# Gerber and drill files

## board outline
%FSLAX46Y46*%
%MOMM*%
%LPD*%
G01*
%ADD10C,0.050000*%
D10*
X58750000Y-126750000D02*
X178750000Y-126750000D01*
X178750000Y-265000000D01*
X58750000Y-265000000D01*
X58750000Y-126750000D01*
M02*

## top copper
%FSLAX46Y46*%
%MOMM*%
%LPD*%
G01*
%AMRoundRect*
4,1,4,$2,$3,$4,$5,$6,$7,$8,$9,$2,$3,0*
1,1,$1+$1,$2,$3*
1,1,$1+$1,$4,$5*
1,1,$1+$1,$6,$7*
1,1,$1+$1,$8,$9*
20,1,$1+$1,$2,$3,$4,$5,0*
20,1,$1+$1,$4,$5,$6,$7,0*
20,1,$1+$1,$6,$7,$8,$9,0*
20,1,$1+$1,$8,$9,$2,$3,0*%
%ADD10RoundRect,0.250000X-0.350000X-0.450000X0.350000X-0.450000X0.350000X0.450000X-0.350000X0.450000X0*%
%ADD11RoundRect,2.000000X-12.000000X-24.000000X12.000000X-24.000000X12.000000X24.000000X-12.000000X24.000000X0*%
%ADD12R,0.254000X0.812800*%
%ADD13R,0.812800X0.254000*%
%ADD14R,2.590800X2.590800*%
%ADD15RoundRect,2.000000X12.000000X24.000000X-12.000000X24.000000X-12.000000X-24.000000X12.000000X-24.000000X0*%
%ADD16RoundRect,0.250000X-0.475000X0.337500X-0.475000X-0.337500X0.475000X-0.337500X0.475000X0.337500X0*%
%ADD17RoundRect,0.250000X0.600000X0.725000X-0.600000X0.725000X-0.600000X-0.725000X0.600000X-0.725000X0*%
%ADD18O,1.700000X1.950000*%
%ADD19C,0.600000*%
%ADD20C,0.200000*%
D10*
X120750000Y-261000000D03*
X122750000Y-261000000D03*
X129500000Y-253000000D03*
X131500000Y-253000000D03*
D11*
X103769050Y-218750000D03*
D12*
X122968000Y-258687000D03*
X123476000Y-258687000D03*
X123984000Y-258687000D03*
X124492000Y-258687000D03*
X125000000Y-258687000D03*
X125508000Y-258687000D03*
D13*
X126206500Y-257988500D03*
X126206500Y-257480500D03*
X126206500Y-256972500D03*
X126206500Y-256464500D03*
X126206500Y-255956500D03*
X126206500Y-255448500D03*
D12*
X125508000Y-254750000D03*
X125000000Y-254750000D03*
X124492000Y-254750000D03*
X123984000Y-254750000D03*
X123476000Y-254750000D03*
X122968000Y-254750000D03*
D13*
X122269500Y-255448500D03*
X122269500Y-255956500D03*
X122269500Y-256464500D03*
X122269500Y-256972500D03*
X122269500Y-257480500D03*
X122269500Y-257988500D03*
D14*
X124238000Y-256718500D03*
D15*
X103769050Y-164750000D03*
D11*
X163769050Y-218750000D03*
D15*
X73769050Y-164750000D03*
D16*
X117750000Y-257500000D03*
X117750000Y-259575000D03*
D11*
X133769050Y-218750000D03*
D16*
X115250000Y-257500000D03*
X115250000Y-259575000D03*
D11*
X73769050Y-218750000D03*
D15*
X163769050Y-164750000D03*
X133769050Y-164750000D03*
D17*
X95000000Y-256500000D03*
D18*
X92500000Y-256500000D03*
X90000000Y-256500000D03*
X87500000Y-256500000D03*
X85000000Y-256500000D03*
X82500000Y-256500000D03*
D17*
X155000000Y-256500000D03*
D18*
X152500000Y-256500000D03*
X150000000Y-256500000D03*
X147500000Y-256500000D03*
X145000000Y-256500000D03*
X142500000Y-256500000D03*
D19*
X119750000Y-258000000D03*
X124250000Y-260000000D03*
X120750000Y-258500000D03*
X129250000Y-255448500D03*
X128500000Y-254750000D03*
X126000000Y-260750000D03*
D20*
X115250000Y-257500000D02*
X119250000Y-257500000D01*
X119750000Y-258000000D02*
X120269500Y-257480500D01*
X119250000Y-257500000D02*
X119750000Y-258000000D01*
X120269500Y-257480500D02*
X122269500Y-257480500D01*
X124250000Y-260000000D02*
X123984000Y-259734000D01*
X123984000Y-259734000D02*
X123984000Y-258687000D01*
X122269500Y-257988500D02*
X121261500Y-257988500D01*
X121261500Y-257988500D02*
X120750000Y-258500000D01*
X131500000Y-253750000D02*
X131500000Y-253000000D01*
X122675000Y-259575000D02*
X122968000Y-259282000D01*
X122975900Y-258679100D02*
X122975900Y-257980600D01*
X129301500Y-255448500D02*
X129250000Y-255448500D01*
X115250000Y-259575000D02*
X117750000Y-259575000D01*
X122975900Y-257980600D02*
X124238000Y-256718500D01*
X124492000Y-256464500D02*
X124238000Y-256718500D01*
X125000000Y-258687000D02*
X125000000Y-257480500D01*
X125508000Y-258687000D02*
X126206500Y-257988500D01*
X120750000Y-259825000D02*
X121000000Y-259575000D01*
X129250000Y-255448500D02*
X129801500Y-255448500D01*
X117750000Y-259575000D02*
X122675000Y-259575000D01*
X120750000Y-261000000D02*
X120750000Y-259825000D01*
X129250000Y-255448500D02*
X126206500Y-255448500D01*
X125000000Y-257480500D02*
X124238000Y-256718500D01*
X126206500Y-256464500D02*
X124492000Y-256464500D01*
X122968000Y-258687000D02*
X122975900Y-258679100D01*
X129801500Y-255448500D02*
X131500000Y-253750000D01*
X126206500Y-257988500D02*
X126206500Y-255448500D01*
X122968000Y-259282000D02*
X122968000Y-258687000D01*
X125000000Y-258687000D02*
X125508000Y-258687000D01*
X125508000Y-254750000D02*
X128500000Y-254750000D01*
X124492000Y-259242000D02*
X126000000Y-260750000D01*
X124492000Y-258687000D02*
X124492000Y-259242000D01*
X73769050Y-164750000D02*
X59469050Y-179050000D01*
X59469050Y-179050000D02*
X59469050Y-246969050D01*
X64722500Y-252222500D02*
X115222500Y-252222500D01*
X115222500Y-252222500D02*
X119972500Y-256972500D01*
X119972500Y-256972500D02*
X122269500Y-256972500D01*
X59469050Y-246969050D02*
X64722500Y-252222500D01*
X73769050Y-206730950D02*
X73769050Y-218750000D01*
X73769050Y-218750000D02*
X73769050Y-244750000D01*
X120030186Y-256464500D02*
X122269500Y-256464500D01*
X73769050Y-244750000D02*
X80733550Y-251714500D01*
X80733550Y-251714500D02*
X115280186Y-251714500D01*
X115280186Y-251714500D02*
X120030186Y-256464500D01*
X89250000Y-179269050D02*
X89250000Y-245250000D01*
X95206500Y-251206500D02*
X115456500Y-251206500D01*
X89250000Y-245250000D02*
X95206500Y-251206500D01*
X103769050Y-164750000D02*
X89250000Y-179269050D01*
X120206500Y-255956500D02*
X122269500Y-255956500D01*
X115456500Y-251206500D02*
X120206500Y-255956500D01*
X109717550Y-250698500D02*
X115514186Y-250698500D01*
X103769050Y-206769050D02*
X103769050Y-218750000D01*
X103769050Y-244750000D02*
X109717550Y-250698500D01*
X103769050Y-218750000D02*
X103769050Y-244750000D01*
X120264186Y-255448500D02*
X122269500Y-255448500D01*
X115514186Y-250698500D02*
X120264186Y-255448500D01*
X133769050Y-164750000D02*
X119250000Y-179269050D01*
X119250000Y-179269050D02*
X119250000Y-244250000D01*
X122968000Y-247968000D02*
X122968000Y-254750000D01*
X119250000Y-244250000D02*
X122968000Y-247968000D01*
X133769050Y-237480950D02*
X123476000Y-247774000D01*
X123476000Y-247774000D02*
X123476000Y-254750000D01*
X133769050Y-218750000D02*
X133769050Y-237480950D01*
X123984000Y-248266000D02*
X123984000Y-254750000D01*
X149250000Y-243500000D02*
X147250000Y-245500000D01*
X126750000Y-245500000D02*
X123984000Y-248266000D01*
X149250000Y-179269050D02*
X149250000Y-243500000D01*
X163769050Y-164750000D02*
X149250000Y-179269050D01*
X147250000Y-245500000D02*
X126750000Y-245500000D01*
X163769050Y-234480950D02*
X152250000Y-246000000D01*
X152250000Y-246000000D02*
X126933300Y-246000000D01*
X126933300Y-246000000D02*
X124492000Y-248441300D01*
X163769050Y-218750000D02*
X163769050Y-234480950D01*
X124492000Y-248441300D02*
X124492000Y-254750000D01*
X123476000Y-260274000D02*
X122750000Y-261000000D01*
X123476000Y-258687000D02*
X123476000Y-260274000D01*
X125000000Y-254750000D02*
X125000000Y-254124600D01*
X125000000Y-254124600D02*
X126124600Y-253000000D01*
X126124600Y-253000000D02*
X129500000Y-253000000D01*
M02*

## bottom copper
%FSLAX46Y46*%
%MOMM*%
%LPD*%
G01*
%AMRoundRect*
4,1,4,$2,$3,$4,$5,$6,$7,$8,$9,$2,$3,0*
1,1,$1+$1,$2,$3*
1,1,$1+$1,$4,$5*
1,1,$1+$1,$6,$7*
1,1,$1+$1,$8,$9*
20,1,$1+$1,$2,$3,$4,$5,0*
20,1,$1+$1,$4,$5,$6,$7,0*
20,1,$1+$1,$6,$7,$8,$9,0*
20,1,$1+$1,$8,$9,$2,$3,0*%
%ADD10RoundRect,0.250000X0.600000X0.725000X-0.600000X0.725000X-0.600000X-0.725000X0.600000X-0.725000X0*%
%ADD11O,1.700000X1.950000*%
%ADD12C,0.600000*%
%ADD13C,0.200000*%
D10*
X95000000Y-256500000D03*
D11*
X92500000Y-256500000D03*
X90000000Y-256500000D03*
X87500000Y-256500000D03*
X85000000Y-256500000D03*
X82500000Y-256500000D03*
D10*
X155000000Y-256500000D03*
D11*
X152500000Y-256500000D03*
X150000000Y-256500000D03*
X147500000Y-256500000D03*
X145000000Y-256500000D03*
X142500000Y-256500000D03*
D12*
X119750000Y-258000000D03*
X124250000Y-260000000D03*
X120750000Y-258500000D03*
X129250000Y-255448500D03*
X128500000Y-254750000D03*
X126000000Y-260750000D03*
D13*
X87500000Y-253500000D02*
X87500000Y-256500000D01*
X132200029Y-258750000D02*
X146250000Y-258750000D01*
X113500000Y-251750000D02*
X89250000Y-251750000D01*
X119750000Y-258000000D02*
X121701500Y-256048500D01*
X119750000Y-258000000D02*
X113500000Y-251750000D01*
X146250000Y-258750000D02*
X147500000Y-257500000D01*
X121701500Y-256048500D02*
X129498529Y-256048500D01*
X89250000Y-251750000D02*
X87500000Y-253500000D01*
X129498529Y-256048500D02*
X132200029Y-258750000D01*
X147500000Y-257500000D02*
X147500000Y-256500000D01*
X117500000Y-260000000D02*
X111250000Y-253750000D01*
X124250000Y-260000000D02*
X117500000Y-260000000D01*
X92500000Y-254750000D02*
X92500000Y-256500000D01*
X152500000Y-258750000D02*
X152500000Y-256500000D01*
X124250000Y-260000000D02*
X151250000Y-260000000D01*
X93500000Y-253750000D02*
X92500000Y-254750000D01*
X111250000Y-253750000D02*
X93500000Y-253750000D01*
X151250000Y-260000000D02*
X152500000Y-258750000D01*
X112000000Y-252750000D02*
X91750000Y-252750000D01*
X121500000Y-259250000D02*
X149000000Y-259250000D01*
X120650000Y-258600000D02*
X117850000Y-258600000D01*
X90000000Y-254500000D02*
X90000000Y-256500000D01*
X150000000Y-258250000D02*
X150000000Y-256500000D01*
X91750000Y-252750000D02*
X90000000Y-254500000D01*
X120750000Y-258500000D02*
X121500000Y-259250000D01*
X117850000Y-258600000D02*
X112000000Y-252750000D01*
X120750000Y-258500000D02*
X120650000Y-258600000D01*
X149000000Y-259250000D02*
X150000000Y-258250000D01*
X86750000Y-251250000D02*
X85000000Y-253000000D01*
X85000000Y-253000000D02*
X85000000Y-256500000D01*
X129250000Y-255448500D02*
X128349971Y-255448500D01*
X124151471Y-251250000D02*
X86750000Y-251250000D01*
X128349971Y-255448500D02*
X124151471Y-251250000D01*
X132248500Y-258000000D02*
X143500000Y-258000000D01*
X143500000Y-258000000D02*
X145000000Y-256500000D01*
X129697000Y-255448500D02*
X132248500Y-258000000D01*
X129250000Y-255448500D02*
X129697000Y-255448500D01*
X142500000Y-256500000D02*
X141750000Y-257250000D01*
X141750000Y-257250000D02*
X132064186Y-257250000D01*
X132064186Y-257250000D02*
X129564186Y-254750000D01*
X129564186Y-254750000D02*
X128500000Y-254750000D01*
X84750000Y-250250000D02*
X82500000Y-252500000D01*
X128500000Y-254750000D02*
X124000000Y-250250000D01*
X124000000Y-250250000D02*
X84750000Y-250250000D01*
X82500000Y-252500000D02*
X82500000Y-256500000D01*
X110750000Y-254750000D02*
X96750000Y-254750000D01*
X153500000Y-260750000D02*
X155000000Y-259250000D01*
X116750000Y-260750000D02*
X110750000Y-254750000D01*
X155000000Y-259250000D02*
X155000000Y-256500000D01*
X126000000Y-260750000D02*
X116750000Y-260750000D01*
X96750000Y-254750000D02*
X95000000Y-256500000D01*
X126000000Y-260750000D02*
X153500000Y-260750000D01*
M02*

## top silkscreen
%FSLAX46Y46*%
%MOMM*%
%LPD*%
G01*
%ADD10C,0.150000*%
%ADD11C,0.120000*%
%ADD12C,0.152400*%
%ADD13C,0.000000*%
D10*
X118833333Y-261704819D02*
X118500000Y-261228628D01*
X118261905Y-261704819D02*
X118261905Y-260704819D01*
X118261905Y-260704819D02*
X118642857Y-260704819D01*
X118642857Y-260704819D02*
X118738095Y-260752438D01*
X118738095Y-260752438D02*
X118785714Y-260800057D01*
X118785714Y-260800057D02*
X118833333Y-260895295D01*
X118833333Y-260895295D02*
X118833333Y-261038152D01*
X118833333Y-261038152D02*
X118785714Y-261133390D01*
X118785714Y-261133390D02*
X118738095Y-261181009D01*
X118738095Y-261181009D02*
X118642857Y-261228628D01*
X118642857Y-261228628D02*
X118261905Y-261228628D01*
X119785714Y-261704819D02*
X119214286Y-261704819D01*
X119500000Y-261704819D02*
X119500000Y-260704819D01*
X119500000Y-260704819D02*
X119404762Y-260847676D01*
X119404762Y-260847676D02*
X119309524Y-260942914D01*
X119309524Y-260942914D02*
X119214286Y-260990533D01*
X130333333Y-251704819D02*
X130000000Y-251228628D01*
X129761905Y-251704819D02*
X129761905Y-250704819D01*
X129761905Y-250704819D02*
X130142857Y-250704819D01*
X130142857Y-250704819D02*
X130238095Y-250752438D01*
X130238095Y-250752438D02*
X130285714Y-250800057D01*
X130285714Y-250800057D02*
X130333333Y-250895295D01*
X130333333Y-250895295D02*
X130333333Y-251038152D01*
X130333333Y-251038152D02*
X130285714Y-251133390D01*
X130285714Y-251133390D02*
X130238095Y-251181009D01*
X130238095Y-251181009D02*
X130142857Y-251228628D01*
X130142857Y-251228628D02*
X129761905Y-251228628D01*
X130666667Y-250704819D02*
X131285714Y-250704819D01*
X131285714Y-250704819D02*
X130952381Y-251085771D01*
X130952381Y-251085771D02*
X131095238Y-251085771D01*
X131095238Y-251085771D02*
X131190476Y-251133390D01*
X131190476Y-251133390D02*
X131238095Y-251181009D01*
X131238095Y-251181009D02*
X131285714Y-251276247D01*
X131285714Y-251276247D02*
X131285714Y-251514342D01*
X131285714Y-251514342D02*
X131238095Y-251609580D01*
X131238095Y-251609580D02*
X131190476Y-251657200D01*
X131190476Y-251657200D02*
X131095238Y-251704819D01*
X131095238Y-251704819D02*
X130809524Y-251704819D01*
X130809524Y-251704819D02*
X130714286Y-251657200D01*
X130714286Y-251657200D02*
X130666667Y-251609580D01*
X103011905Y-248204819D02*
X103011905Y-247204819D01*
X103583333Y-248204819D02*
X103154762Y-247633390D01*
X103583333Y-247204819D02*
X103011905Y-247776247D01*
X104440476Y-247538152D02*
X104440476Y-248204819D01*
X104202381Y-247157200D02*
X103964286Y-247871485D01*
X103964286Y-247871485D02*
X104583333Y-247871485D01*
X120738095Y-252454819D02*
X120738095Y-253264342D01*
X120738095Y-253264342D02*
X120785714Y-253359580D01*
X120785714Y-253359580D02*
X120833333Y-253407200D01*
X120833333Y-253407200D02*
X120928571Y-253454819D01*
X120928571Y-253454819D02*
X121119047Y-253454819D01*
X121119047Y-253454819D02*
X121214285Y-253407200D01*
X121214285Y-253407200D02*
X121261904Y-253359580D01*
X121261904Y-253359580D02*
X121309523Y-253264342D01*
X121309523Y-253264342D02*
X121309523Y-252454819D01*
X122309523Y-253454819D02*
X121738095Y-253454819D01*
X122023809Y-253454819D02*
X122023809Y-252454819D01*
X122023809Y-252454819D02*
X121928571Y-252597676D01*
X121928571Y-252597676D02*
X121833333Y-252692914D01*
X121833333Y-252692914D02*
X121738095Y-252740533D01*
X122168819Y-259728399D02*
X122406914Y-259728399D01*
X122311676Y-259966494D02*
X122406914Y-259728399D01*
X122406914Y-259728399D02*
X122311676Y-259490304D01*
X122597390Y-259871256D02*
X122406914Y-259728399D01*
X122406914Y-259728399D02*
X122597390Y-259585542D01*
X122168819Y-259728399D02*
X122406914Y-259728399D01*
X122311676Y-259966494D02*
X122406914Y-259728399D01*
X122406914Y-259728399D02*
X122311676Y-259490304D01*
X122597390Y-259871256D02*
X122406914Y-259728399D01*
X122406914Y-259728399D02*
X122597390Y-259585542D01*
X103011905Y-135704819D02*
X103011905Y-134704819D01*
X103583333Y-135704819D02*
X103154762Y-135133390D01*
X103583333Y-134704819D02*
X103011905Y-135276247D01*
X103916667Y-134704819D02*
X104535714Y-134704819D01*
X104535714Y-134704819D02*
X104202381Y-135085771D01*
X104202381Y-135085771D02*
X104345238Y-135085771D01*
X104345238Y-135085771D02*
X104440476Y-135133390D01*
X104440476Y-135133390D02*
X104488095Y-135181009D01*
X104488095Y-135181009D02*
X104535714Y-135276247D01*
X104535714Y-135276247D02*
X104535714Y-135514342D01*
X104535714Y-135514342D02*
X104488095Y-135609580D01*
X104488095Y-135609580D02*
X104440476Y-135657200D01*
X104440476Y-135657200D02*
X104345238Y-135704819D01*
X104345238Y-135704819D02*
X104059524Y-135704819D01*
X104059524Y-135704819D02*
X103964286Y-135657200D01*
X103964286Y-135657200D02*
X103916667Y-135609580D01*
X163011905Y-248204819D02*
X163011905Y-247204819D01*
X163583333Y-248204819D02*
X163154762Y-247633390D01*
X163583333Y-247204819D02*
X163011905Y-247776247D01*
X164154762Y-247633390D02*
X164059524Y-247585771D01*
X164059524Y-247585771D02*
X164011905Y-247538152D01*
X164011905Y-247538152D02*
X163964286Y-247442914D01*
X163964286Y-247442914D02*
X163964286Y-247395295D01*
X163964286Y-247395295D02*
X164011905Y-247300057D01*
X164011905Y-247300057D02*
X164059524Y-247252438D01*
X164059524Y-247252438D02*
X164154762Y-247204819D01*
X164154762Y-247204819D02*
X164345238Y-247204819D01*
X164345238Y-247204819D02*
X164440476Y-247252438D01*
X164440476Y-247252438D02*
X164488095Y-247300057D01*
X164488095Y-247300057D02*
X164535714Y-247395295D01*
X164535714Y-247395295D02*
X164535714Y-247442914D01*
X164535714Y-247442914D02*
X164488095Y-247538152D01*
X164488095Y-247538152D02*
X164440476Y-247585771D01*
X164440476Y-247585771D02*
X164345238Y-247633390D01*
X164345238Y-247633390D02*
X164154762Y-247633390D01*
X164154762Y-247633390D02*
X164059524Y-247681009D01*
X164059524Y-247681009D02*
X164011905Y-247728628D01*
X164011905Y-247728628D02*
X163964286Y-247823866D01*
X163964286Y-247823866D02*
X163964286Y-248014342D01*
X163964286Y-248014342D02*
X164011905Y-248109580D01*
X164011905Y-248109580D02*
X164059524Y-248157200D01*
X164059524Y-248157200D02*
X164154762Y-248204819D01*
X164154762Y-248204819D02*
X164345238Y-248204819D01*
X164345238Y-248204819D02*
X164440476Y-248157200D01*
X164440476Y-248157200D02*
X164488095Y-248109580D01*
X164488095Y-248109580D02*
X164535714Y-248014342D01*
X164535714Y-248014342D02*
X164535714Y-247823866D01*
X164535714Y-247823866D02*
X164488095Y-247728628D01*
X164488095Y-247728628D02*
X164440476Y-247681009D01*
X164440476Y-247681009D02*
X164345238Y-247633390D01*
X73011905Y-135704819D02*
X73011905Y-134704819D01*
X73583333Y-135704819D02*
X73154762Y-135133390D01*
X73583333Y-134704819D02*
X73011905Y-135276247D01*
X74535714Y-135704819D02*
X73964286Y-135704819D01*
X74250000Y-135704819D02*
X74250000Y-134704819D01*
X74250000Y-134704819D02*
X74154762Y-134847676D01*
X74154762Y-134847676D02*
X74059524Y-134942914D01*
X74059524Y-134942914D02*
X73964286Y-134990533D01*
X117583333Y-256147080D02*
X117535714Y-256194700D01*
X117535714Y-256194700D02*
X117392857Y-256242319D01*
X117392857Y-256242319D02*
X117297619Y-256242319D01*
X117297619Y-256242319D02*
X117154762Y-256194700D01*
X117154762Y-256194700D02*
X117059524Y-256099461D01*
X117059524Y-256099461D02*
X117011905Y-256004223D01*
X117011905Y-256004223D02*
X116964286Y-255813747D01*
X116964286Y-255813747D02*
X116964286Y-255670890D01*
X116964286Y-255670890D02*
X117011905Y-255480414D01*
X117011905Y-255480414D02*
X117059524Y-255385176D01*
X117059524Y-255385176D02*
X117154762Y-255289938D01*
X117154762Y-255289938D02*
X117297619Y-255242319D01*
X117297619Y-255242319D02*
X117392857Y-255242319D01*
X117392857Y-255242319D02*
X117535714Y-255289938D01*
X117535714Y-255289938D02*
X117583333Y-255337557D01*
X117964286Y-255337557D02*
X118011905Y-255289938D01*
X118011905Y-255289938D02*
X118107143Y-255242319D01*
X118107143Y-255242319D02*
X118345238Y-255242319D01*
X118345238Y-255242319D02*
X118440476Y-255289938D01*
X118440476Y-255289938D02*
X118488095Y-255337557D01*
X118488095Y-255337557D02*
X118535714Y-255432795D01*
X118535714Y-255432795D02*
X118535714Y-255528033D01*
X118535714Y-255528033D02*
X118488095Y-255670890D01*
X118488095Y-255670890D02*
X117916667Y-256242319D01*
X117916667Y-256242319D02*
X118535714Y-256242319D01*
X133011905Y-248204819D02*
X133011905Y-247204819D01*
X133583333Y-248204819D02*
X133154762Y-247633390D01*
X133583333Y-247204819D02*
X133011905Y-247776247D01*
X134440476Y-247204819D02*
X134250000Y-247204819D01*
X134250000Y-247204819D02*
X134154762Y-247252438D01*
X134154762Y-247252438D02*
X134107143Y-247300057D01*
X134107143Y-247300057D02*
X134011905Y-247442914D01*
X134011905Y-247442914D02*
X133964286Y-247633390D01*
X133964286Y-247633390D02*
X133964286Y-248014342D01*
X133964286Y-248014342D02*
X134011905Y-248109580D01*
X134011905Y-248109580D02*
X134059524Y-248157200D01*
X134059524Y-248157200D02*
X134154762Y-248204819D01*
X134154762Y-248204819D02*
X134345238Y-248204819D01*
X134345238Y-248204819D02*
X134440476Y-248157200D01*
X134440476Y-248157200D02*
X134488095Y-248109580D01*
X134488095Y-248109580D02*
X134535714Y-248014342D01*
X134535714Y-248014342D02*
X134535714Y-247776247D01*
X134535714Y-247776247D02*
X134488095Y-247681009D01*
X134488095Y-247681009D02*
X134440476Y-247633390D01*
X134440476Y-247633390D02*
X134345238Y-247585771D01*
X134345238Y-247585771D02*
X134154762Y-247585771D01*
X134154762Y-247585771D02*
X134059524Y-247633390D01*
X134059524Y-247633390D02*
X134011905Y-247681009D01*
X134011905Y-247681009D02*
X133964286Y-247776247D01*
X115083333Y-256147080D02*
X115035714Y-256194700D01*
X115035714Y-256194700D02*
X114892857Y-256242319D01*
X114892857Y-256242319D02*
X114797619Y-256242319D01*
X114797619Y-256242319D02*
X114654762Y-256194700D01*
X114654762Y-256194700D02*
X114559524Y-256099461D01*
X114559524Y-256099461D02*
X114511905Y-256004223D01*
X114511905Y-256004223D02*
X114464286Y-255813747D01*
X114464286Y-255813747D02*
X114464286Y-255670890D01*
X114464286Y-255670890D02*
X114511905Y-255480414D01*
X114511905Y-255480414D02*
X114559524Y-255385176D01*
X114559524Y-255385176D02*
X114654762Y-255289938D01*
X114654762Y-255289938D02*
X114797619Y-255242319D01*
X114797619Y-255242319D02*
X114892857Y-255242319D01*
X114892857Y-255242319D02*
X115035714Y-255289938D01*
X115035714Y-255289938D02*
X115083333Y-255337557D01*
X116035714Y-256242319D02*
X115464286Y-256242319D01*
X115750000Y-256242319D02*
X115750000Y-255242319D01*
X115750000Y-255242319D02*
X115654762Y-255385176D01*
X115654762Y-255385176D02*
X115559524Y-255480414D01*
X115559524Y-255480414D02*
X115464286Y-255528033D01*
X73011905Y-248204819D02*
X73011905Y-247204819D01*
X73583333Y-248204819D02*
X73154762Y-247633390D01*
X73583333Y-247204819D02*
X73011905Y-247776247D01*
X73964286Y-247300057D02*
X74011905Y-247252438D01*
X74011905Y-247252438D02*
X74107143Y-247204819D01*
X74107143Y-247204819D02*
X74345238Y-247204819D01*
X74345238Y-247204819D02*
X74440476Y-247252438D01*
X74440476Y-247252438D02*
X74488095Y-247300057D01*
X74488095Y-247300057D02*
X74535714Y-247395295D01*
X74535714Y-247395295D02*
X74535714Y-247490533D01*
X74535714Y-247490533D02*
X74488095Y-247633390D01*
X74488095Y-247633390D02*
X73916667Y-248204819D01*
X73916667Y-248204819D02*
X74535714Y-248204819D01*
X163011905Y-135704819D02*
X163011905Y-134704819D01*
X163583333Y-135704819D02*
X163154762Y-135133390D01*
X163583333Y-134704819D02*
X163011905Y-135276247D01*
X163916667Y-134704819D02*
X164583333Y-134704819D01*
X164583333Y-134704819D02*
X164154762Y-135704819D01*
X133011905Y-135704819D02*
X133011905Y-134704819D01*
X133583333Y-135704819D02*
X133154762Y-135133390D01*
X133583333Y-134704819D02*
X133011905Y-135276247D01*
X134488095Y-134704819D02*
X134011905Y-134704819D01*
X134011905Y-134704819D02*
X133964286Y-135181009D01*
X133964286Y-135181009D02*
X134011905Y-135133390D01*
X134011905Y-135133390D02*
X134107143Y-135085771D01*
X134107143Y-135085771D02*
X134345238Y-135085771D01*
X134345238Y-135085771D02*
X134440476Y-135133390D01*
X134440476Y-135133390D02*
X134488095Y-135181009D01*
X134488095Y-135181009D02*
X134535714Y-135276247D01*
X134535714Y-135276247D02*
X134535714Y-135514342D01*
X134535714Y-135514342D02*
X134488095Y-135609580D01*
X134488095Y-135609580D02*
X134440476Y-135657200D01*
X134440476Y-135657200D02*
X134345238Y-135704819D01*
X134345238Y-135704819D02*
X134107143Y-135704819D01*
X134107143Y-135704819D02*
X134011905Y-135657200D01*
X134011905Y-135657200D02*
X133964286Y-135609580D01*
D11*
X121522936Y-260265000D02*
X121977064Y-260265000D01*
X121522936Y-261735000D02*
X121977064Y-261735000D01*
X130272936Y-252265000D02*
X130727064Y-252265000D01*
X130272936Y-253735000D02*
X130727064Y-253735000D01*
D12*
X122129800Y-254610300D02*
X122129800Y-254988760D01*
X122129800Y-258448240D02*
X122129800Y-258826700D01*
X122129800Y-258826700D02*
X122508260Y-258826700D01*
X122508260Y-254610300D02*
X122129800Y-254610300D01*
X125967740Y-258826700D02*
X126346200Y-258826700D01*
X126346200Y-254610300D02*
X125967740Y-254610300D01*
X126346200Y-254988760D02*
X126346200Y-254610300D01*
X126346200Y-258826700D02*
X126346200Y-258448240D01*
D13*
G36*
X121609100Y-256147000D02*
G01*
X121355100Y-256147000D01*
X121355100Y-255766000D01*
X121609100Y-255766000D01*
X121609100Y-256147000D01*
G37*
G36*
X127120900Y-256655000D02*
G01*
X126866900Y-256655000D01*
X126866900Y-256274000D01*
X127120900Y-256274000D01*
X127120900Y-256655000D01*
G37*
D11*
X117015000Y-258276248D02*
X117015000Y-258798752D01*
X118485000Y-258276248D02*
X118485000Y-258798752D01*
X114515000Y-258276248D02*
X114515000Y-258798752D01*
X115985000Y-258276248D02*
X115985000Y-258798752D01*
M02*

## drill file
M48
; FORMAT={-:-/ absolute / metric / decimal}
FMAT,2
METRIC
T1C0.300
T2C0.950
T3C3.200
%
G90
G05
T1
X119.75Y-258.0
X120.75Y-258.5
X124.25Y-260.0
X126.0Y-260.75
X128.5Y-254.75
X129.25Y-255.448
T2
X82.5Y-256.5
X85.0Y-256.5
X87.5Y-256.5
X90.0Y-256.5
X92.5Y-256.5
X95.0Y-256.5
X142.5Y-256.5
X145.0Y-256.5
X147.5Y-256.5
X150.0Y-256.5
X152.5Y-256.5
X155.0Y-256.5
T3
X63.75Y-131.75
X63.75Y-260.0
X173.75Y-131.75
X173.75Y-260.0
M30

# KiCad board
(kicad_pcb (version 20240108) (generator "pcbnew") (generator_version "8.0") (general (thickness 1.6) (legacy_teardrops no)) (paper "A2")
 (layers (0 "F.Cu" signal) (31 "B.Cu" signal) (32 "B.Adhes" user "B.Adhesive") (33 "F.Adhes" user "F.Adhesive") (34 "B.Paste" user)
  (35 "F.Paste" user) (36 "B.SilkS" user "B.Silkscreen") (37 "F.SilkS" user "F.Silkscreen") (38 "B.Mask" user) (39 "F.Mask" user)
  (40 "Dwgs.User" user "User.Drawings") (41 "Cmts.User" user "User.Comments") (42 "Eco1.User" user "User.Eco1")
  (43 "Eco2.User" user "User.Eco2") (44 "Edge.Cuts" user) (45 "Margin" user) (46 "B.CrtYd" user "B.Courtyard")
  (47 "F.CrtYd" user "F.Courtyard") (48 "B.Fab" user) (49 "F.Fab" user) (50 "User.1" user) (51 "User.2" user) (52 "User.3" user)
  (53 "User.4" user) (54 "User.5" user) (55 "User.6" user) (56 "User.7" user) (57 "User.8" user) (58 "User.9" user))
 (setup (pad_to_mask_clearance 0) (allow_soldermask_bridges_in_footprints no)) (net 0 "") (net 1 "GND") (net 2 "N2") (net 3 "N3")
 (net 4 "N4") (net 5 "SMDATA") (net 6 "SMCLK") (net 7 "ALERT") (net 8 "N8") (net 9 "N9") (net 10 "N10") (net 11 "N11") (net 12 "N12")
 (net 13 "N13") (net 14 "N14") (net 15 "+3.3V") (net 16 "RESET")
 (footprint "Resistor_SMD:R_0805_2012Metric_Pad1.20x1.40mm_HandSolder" (layer "F.Cu") (at 121.75 261)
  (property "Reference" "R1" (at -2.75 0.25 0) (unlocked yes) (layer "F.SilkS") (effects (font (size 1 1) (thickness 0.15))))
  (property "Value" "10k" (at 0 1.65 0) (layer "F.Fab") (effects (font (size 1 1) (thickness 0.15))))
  (fp_line (start -0.227064 -0.735) (end 0.227064 -0.735) (stroke (width 0.12) (type solid)) (layer "F.SilkS"))
  (fp_line (start -0.227064 0.735) (end 0.227064 0.735) (stroke (width 0.12) (type solid)) (layer "F.SilkS"))
  (pad "1" smd roundrect (at -1 0) (size 1.2 1.4) (layers "F.Cu" "F.Paste" "F.Mask") (roundrect_rratio 0.208333) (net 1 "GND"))
  (pad "2" smd roundrect (at 1 0) (size 1.2 1.4) (layers "F.Cu" "F.Paste" "F.Mask") (roundrect_rratio 0.208333) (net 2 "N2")))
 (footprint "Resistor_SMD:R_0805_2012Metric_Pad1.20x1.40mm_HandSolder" (layer "F.Cu") (at 130.5 253)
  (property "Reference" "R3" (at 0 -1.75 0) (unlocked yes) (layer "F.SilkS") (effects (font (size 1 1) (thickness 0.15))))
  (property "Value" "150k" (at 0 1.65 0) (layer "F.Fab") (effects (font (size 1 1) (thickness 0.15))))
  (fp_line (start -0.227064 -0.735) (end 0.227064 -0.735) (stroke (width 0.12) (type solid)) (layer "F.SilkS"))
  (fp_line (start -0.227064 0.735) (end 0.227064 0.735) (stroke (width 0.12) (type solid)) (layer "F.SilkS"))
  (pad "1" smd roundrect (at -1 0) (size 1.2 1.4) (layers "F.Cu" "F.Paste" "F.Mask") (roundrect_rratio 0.208333) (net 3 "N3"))
  (pad "2" smd roundrect (at 1 0) (size 1.2 1.4) (layers "F.Cu" "F.Paste" "F.Mask") (roundrect_rratio 0.208333) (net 1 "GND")))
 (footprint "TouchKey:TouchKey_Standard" (layer "F.Cu") (at 103.76905 218.75)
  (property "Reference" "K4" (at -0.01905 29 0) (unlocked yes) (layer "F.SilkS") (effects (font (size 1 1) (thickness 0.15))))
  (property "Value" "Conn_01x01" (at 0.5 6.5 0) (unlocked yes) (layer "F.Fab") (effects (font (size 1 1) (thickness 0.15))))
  (pad "1" smd roundrect (at 0 0) (size 28 52) (layers "F.Cu") (roundrect_rratio 0.07142857143) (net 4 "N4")))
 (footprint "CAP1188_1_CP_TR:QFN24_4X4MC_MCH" (layer "F.Cu") (at 124.238 256.7185 90)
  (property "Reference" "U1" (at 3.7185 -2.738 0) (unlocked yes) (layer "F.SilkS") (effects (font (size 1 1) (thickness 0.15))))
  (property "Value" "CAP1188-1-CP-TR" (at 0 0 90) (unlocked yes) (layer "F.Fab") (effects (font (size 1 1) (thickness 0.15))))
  (fp_line (start 2.1082 -2.1082) (end 1.72974 -2.1082) (stroke (width 0.1524) (type solid)) (layer "F.SilkS"))
  (fp_line (start -1.72974 -2.1082) (end -2.1082 -2.1082) (stroke (width 0.1524) (type solid)) (layer "F.SilkS"))
  (fp_line (start -2.1082 -2.1082) (end -2.1082 -1.72974) (stroke (width 0.1524) (type solid)) (layer "F.SilkS"))
  (fp_line (start 2.1082 -1.72974) (end 2.1082 -2.1082) (stroke (width 0.1524) (type solid)) (layer "F.SilkS"))
  (fp_line (start -2.1082 1.72974) (end -2.1082 2.1082) (stroke (width 0.1524) (type solid)) (layer "F.SilkS"))
  (fp_line (start 2.1082 2.1082) (end 2.1082 1.72974) (stroke (width 0.1524) (type solid)) (layer "F.SilkS"))
  (fp_line (start 1.72974 2.1082) (end 2.1082 2.1082) (stroke (width 0.1524) (type solid)) (layer "F.SilkS"))
  (fp_line (start -2.1082 2.1082) (end -1.72974 2.1082) (stroke (width 0.1524) (type solid)) (layer "F.SilkS"))
  (fp_poly
   (pts (xy 0.5715 -2.6289) (xy 0.5715 -2.8829) (xy 0.9525 -2.8829) (xy 0.9525 -2.6289)) (stroke (width 0) (type solid)) (fill solid)
   (layer "F.SilkS"))
  (fp_poly
   (pts (xy 0.0635 2.6289) (xy 0.0635 2.8829) (xy 0.4445 2.8829) (xy 0.4445 2.6289)) (stroke (width 0) (type solid)) (fill solid)
   (layer "F.SilkS"))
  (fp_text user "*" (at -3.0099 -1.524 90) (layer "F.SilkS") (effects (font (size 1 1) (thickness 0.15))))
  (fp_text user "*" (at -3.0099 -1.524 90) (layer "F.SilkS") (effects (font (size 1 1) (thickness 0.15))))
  (pad "1" smd rect (at -1.9685 -1.27 180) (size 0.254 0.8128) (layers "F.Cu" "F.Paste" "F.Mask") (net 1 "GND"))
  (pad "2" smd rect (at -1.9685 -0.762 180) (size 0.254 0.8128) (layers "F.Cu" "F.Paste" "F.Mask") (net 2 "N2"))
  (pad "3" smd rect (at -1.9685 -0.254 180) (size 0.254 0.8128) (layers "F.Cu" "F.Paste" "F.Mask") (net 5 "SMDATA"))
  (pad "4" smd rect (at -1.9685 0.254 180) (size 0.254 0.8128) (layers "F.Cu" "F.Paste" "F.Mask") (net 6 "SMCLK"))
  (pad "5" smd rect (at -1.9685 0.762 180) (size 0.254 0.8128) (layers "F.Cu" "F.Paste" "F.Mask") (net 1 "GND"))
  (pad "6" smd rect (at -1.9685 1.27 180) (size 0.254 0.8128) (layers "F.Cu" "F.Paste" "F.Mask") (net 1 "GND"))
  (pad "7" smd rect (at -1.27 1.9685 90) (size 0.254 0.8128) (layers "F.Cu" "F.Paste" "F.Mask") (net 1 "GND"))
  (pad "8" smd rect (at -0.762 1.9685 90) (size 0.254 0.8128) (layers "F.Cu" "F.Paste" "F.Mask") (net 1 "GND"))
  (pad "9" smd rect (at -0.254 1.9685 90) (size 0.254 0.8128) (layers "F.Cu" "F.Paste" "F.Mask") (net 1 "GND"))
  (pad "10" smd rect (at 0.254 1.9685 90) (size 0.254 0.8128) (layers "F.Cu" "F.Paste" "F.Mask") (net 1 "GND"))
  (pad "11" smd rect (at 0.762 1.9685 90) (size 0.254 0.8128) (layers "F.Cu" "F.Paste" "F.Mask") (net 1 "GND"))
  (pad "12" smd rect (at 1.27 1.9685 90) (size 0.254 0.8128) (layers "F.Cu" "F.Paste" "F.Mask") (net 1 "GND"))
  (pad "13" smd rect (at 1.9685 1.27 180) (size 0.254 0.8128) (layers "F.Cu" "F.Paste" "F.Mask") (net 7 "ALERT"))
  (pad "14" smd rect (at 1.9685 0.762 180) (size 0.254 0.8128) (layers "F.Cu" "F.Paste" "F.Mask") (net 3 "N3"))
  (pad "15" smd rect (at 1.9685 0.254 180) (size 0.254 0.8128) (layers "F.Cu" "F.Paste" "F.Mask") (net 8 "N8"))
  (pad "16" smd rect (at 1.9685 -0.254 180) (size 0.254 0.8128) (layers "F.Cu" "F.Paste" "F.Mask") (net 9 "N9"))
  (pad "17" smd rect (at 1.9685 -0.762 180) (size 0.254 0.8128) (layers "F.Cu" "F.Paste" "F.Mask") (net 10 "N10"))
  (pad "18" smd rect (at 1.9685 -1.27 180) (size 0.254 0.8128) (layers "F.Cu" "F.Paste" "F.Mask") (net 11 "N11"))
  (pad "19" smd rect (at 1.27 -1.9685 90) (size 0.254 0.8128) (layers "F.Cu" "F.Paste" "F.Mask") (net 4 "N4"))
  (pad "20" smd rect (at 0.762 -1.9685 90) (size 0.254 0.8128) (layers "F.Cu" "F.Paste" "F.Mask") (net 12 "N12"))
  (pad "21" smd rect (at 0.254 -1.9685 90) (size 0.254 0.8128) (layers "F.Cu" "F.Paste" "F.Mask") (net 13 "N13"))
  (pad "22" smd rect (at -0.254 -1.9685 90) (size 0.254 0.8128) (layers "F.Cu" "F.Paste" "F.Mask") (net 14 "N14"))
  (pad "23" smd rect (at -0.762 -1.9685 90) (size 0.254 0.8128) (layers "F.Cu" "F.Paste" "F.Mask") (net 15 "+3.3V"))
  (pad "24" smd rect (at -1.27 -1.9685 90) (size 0.254 0.8128) (layers "F.Cu" "F.Paste" "F.Mask") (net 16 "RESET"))
  (pad "25" smd rect (at 0 0 90) (size 2.5908 2.5908) (layers "F.Cu" "F.Paste" "F.Mask") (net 1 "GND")))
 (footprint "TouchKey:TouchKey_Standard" (layer "F.Cu") (at 103.76905 164.75 180)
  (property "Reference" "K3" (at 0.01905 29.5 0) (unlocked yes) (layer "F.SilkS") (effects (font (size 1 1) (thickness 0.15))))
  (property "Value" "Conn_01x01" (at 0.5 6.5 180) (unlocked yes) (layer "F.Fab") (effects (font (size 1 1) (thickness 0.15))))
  (pad "1" smd roundrect (at 0 0 180) (size 28 52) (layers "F.Cu") (roundrect_rratio 0.07142857143) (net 12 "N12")))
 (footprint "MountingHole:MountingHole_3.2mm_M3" (layer "F.Cu") (at 173.75 131.75)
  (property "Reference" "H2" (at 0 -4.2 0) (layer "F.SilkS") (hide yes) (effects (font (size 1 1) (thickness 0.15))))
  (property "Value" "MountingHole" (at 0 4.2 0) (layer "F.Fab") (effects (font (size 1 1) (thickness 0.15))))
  (pad "" np_thru_hole circle (at 0 0) (size 3.2 3.2) (drill 3.2) (layers "*.Cu" "*.Mask")))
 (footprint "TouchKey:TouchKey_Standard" (layer "F.Cu") (at 163.76905 218.75)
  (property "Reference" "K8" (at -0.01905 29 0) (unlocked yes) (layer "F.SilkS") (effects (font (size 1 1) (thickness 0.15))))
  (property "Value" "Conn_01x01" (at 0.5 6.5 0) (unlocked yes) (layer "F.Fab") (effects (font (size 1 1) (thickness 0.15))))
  (pad "1" smd roundrect (at 0 0) (size 28 52) (layers "F.Cu") (roundrect_rratio 0.07142857143) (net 8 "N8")))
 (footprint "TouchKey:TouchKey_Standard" (layer "F.Cu") (at 73.76905 164.75 180)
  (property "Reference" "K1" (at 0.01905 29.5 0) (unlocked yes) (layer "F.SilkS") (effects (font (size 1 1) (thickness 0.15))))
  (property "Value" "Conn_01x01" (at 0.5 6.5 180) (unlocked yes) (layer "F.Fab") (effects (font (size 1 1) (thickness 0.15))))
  (pad "1" smd roundrect (at 0 0 180) (size 28 52) (layers "F.Cu") (roundrect_rratio 0.07142857143) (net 14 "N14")))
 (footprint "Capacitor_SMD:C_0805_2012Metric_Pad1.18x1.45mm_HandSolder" (layer "F.Cu") (at 117.75 258.5375 -90)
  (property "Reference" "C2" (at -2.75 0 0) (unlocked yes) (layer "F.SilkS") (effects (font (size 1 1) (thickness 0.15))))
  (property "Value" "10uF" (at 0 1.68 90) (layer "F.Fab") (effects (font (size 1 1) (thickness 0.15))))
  (fp_line (start -0.261252 0.735) (end 0.261252 0.735) (stroke (width 0.12) (type solid)) (layer "F.SilkS"))
  (fp_line (start -0.261252 -0.735) (end 0.261252 -0.735) (stroke (width 0.12) (type solid)) (layer "F.SilkS"))
  (pad "1" smd roundrect (at -1.0375 0 270) (size 1.175 1.45) (layers "F.Cu" "F.Paste" "F.Mask") (roundrect_rratio 0.212766)
   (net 15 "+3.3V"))
  (pad "2" smd roundrect (at 1.0375 0 270) (size 1.175 1.45) (layers "F.Cu" "F.Paste" "F.Mask") (roundrect_rratio 0.212766) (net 1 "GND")))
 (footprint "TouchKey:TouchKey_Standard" (layer "F.Cu") (at 133.76905 218.75)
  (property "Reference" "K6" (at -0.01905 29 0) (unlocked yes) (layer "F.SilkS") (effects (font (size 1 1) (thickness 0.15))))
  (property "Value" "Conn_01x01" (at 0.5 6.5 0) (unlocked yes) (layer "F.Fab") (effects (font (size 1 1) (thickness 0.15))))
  (pad "1" smd roundrect (at 0 0) (size 28 52) (layers "F.Cu") (roundrect_rratio 0.07142857143) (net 10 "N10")))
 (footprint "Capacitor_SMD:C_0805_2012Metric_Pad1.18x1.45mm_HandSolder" (layer "F.Cu") (at 115.25 258.5375 -90)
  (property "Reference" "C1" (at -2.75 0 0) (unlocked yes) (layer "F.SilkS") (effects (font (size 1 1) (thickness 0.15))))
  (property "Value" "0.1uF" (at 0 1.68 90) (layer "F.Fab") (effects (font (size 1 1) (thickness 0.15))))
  (fp_line (start -0.261252 0.735) (end 0.261252 0.735) (stroke (width 0.12) (type solid)) (layer "F.SilkS"))
  (fp_line (start -0.261252 -0.735) (end 0.261252 -0.735) (stroke (width 0.12) (type solid)) (layer "F.SilkS"))
  (pad "1" smd roundrect (at -1.0375 0 270) (size 1.175 1.45) (layers "F.Cu" "F.Paste" "F.Mask") (roundrect_rratio 0.212766)
   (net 15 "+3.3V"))
  (pad "2" smd roundrect (at 1.0375 0 270) (size 1.175 1.45) (layers "F.Cu" "F.Paste" "F.Mask") (roundrect_rratio 0.212766) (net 1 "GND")))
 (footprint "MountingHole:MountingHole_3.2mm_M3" (layer "F.Cu") (at 63.75 260)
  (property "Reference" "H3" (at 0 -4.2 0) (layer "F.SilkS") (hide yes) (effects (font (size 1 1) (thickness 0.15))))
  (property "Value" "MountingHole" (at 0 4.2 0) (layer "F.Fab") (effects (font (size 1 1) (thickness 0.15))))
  (pad "" np_thru_hole circle (at 0 0) (size 3.2 3.2) (drill 3.2) (layers "*.Cu" "*.Mask")))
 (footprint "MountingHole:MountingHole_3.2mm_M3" (layer "F.Cu") (at 63.75 131.75)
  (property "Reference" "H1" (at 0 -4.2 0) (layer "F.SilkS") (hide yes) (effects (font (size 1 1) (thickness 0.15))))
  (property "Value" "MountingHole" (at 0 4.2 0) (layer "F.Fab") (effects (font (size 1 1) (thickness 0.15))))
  (pad "" np_thru_hole circle (at 0 0) (size 3.2 3.2) (drill 3.2) (layers "*.Cu" "*.Mask")))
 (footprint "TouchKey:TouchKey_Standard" (layer "F.Cu") (at 73.76905 218.75)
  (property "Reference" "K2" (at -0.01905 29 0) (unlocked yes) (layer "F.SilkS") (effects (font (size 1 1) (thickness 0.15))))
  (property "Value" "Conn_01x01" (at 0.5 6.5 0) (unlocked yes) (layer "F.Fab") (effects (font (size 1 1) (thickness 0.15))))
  (pad "1" smd roundrect (at 0 0) (size 28 52) (layers "F.Cu") (roundrect_rratio 0.07142857143) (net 13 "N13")))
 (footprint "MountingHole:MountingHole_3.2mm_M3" (layer "F.Cu") (at 173.75 260)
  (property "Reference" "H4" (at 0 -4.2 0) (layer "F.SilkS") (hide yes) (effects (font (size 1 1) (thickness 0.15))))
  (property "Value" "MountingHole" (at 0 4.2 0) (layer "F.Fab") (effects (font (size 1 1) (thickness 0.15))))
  (pad "" np_thru_hole circle (at 0 0) (size 3.2 3.2) (drill 3.2) (layers "*.Cu" "*.Mask")))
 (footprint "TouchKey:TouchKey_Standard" (layer "F.Cu") (at 163.76905 164.75 180)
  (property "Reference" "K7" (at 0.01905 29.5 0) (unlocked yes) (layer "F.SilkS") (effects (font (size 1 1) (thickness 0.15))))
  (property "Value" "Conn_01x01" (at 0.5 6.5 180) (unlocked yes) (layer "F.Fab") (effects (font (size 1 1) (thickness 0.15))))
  (pad "1" smd roundrect (at 0 0 180) (size 28 52) (layers "F.Cu") (roundrect_rratio 0.07142857143) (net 9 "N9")))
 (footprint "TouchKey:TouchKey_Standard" (layer "F.Cu") (at 133.76905 164.75 180)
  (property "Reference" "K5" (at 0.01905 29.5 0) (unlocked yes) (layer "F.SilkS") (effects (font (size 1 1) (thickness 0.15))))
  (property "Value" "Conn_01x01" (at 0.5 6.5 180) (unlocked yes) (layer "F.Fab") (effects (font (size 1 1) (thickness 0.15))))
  (pad "1" smd roundrect (at 0 0 180) (size 28 52) (layers "F.Cu") (roundrect_rratio 0.07142857143) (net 11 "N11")))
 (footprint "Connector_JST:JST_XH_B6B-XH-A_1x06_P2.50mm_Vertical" (layer "B.Cu") (at 95 256.5 180)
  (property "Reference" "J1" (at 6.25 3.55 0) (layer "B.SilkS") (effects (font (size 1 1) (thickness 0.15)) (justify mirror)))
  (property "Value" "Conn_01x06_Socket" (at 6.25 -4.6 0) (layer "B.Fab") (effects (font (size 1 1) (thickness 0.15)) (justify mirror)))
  (pad "1" thru_hole roundrect (at 0 0 180) (size 1.7 1.95) (drill 0.95) (layers "*.Cu" "*.Mask") (remove_unused_layers no)
   (roundrect_rratio 0.147059) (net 6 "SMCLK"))
  (pad "2" thru_hole oval (at 2.5 0 180) (size 1.7 1.95) (drill 0.95) (layers "*.Cu" "*.Mask") (remove_unused_layers no) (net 5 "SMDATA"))
  (pad "3" thru_hole oval (at 5 0 180) (size 1.7 1.95) (drill 0.95) (layers "*.Cu" "*.Mask") (remove_unused_layers no) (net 16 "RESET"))
  (pad "4" thru_hole oval (at 7.5 0 180) (size 1.7 1.95) (drill 0.95) (layers "*.Cu" "*.Mask") (remove_unused_layers no) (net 15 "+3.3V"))
  (pad "5" thru_hole oval (at 10 0 180) (size 1.7 1.95) (drill 0.95) (layers "*.Cu" "*.Mask") (remove_unused_layers no) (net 1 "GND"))
  (pad "6" thru_hole oval (at 12.5 0 180) (size 1.7 1.95) (drill 0.95) (layers "*.Cu" "*.Mask") (remove_unused_layers no) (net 7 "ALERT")))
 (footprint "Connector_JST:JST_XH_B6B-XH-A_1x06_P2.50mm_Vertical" (layer "B.Cu") (at 155 256.5 180)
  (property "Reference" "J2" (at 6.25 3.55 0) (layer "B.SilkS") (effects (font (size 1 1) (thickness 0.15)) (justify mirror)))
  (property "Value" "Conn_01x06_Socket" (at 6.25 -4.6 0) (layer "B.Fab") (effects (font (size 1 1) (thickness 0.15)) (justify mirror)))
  (pad "1" thru_hole roundrect (at 0 0 180) (size 1.7 1.95) (drill 0.95) (layers "*.Cu" "*.Mask") (remove_unused_layers no)
   (roundrect_rratio 0.147059) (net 6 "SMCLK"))
  (pad "2" thru_hole oval (at 2.5 0 180) (size 1.7 1.95) (drill 0.95) (layers "*.Cu" "*.Mask") (remove_unused_layers no) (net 5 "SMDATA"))
  (pad "3" thru_hole oval (at 5 0 180) (size 1.7 1.95) (drill 0.95) (layers "*.Cu" "*.Mask") (remove_unused_layers no) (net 16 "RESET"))
  (pad "4" thru_hole oval (at 7.5 0 180) (size 1.7 1.95) (drill 0.95) (layers "*.Cu" "*.Mask") (remove_unused_layers no) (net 15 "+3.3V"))
  (pad "5" thru_hole oval (at 10 0 180) (size 1.7 1.95) (drill 0.95) (layers "*.Cu" "*.Mask") (remove_unused_layers no) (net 1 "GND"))
  (pad "6" thru_hole oval (at 12.5 0 180) (size 1.7 1.95) (drill 0.95) (layers "*.Cu" "*.Mask") (remove_unused_layers no) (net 7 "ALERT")))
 (gr_rect (start 58.75 126.75) (end 178.75 265) (stroke (width 0.05) (type default)) (fill none) (layer "Edge.Cuts"))
 (segment (start 115.25 257.5) (end 119.25 257.5) (width 0.2) (layer "F.Cu") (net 15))
 (segment (start 119.75 258) (end 120.2695 257.4805) (width 0.2) (layer "F.Cu") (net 15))
 (segment (start 119.25 257.5) (end 119.75 258) (width 0.2) (layer "F.Cu") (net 15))
 (segment (start 120.2695 257.4805) (end 122.2695 257.4805) (width 0.2) (layer "F.Cu") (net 15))
 (via (at 119.75 258) (size 0.6) (drill 0.3) (layers "F.Cu" "B.Cu") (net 15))
 (segment (start 87.5 253.5) (end 87.5 256.5) (width 0.2) (layer "B.Cu") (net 15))
 (segment (start 132.200029 258.75) (end 146.25 258.75) (width 0.2) (layer "B.Cu") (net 15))
 (segment (start 113.5 251.75) (end 89.25 251.75) (width 0.2) (layer "B.Cu") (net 15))
 (segment (start 119.75 258) (end 121.7015 256.0485) (width 0.2) (layer "B.Cu") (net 15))
 (segment (start 119.75 258) (end 113.5 251.75) (width 0.2) (layer "B.Cu") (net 15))
 (segment (start 146.25 258.75) (end 147.5 257.5) (width 0.2) (layer "B.Cu") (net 15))
 (segment (start 121.7015 256.0485) (end 129.498529 256.0485) (width 0.2) (layer "B.Cu") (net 15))
 (segment (start 89.25 251.75) (end 87.5 253.5) (width 0.2) (layer "B.Cu") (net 15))
 (segment (start 129.498529 256.0485) (end 132.200029 258.75) (width 0.2) (layer "B.Cu") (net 15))
 (segment (start 147.5 257.5) (end 147.5 256.5) (width 0.2) (layer "B.Cu") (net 15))
 (segment (start 124.25 260) (end 123.984 259.734) (width 0.2) (layer "F.Cu") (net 5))
 (segment (start 123.984 259.734) (end 123.984 258.687) (width 0.2) (layer "F.Cu") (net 5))
 (via (at 124.25 260) (size 0.6) (drill 0.3) (layers "F.Cu" "B.Cu") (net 5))
 (segment (start 117.5 260) (end 111.25 253.75) (width 0.2) (layer "B.Cu") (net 5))
 (segment (start 124.25 260) (end 117.5 260) (width 0.2) (layer "B.Cu") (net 5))
 (segment (start 92.5 254.75) (end 92.5 256.5) (width 0.2) (layer "B.Cu") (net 5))
 (segment (start 152.5 258.75) (end 152.5 256.5) (width 0.2) (layer "B.Cu") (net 5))
 (segment (start 124.25 260) (end 151.25 260) (width 0.2) (layer "B.Cu") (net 5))
 (segment (start 93.5 253.75) (end 92.5 254.75) (width 0.2) (layer "B.Cu") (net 5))
 (segment (start 111.25 253.75) (end 93.5 253.75) (width 0.2) (layer "B.Cu") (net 5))
 (segment (start 151.25 260) (end 152.5 258.75) (width 0.2) (layer "B.Cu") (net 5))
 (segment (start 122.2695 257.9885) (end 121.2615 257.9885) (width 0.2) (layer "F.Cu") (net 16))
 (segment (start 121.2615 257.9885) (end 120.75 258.5) (width 0.2) (layer "F.Cu") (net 16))
 (via (at 120.75 258.5) (size 0.6) (drill 0.3) (layers "F.Cu" "B.Cu") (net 16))
 (segment (start 112 252.75) (end 91.75 252.75) (width 0.2) (layer "B.Cu") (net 16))
 (segment (start 121.5 259.25) (end 149 259.25) (width 0.2) (layer "B.Cu") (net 16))
 (segment (start 120.65 258.6) (end 117.85 258.6) (width 0.2) (layer "B.Cu") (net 16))
 (segment (start 90 254.5) (end 90 256.5) (width 0.2) (layer "B.Cu") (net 16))
 (segment (start 150 258.25) (end 150 256.5) (width 0.2) (layer "B.Cu") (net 16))
 (segment (start 91.75 252.75) (end 90 254.5) (width 0.2) (layer "B.Cu") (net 16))
 (segment (start 120.75 258.5) (end 121.5 259.25) (width 0.2) (layer "B.Cu") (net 16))
 (segment (start 117.85 258.6) (end 112 252.75) (width 0.2) (layer "B.Cu") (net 16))
 (segment (start 120.75 258.5) (end 120.65 258.6) (width 0.2) (layer "B.Cu") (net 16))
 (segment (start 149 259.25) (end 150 258.25) (width 0.2) (layer "B.Cu") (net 16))
 (segment (start 131.5 253.75) (end 131.5 253) (width 0.2) (layer "F.Cu") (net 1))
 (segment (start 122.675 259.575) (end 122.968 259.282) (width 0.2) (layer "F.Cu") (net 1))
 (segment (start 122.9759 258.6791) (end 122.9759 257.9806) (width 0.2) (layer "F.Cu") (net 1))
 (segment (start 129.3015 255.4485) (end 129.25 255.4485) (width 0.2) (layer "F.Cu") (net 1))
 (segment (start 115.25 259.575) (end 117.75 259.575) (width 0.2) (layer "F.Cu") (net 1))
 (segment (start 122.9759 257.9806) (end 124.238 256.7185) (width 0.2) (layer "F.Cu") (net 1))
 (segment (start 124.492 256.4645) (end 124.238 256.7185) (width 0.2) (layer "F.Cu") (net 1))
 (segment (start 125 258.687) (end 125 257.4805) (width 0.2) (layer "F.Cu") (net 1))
 (segment (start 125.508 258.687) (end 126.2065 257.9885) (width 0.2) (layer "F.Cu") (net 1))
 (segment (start 120.75 259.825) (end 121 259.575) (width 0.2) (layer "F.Cu") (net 1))
 (segment (start 129.25 255.4485) (end 129.8015 255.4485) (width 0.2) (layer "F.Cu") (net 1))
 (segment (start 117.75 259.575) (end 122.675 259.575) (width 0.2) (layer "F.Cu") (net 1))
 (segment (start 120.75 261) (end 120.75 259.825) (width 0.2) (layer "F.Cu") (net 1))
 (segment (start 129.25 255.4485) (end 126.2065 255.4485) (width 0.2) (layer "F.Cu") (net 1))
 (segment (start 125 257.4805) (end 124.238 256.7185) (width 0.2) (layer "F.Cu") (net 1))
 (segment (start 126.2065 256.4645) (end 124.492 256.4645) (width 0.2) (layer "F.Cu") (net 1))
 (segment (start 122.968 258.687) (end 122.9759 258.6791) (width 0.2) (layer "F.Cu") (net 1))
 (segment (start 129.8015 255.4485) (end 131.5 253.75) (width 0.2) (layer "F.Cu") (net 1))
 (segment (start 126.2065 257.9885) (end 126.2065 255.4485) (width 0.2) (layer "F.Cu") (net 1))
 (segment (start 122.968 259.282) (end 122.968 258.687) (width 0.2) (layer "F.Cu") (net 1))
 (segment (start 125 258.687) (end 125.508 258.687) (width 0.2) (layer "F.Cu") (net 1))
 (via (at 129.25 255.4485) (size 0.6) (drill 0.3) (layers "F.Cu" "B.Cu") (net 1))
 (segment (start 86.75 251.25) (end 85 253) (width 0.2) (layer "B.Cu") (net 1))
 (segment (start 85 253) (end 85 256.5) (width 0.2) (layer "B.Cu") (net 1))
 (segment (start 129.25 255.4485) (end 128.349971 255.4485) (width 0.2) (layer "B.Cu") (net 1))
 (segment (start 124.151471 251.25) (end 86.75 251.25) (width 0.2) (layer "B.Cu") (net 1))
 (segment (start 128.349971 255.4485) (end 124.151471 251.25) (width 0.2) (layer "B.Cu") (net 1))
 (segment (start 132.2485 258) (end 143.5 258) (width 0.2) (layer "B.Cu") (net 1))
 (segment (start 143.5 258) (end 145 256.5) (width 0.2) (layer "B.Cu") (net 1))
 (segment (start 129.697 255.4485) (end 132.2485 258) (width 0.2) (layer "B.Cu") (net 1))
 (segment (start 129.25 255.4485) (end 129.697 255.4485) (width 0.2) (layer "B.Cu") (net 1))
 (segment (start 125.508 254.75) (end 128.5 254.75) (width 0.2) (layer "F.Cu") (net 7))
 (via (at 128.5 254.75) (size 0.6) (drill 0.3) (layers "F.Cu" "B.Cu") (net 7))
 (segment (start 142.5 256.5) (end 141.75 257.25) (width 0.2) (layer "B.Cu") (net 7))
 (segment (start 141.75 257.25) (end 132.064186 257.25) (width 0.2) (layer "B.Cu") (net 7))
 (segment (start 132.064186 257.25) (end 129.564186 254.75) (width 0.2) (layer "B.Cu") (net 7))
 (segment (start 129.564186 254.75) (end 128.5 254.75) (width 0.2) (layer "B.Cu") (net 7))
 (segment (start 84.75 250.25) (end 82.5 252.5) (width 0.2) (layer "B.Cu") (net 7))
 (segment (start 128.5 254.75) (end 124 250.25) (width 0.2) (layer "B.Cu") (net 7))
 (segment (start 124 250.25) (end 84.75 250.25) (width 0.2) (layer "B.Cu") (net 7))
 (segment (start 82.5 252.5) (end 82.5 256.5) (width 0.2) (layer "B.Cu") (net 7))
 (segment (start 124.492 259.242) (end 126 260.75) (width 0.2) (layer "F.Cu") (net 6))
 (segment (start 124.492 258.687) (end 124.492 259.242) (width 0.2) (layer "F.Cu") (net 6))
 (via (at 126 260.75) (size 0.6) (drill 0.3) (layers "F.Cu" "B.Cu") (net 6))
 (segment (start 110.75 254.75) (end 96.75 254.75) (width 0.2) (layer "B.Cu") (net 6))
 (segment (start 153.5 260.75) (end 155 259.25) (width 0.2) (layer "B.Cu") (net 6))
 (segment (start 116.75 260.75) (end 110.75 254.75) (width 0.2) (layer "B.Cu") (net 6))
 (segment (start 155 259.25) (end 155 256.5) (width 0.2) (layer "B.Cu") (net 6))
 (segment (start 126 260.75) (end 116.75 260.75) (width 0.2) (layer "B.Cu") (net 6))
 (segment (start 96.75 254.75) (end 95 256.5) (width 0.2) (layer "B.Cu") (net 6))
 (segment (start 126 260.75) (end 153.5 260.75) (width 0.2) (layer "B.Cu") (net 6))
 (segment (start 73.76905 164.75) (end 59.46905 179.05) (width 0.2) (layer "F.Cu") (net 14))
 (segment (start 59.46905 179.05) (end 59.46905 246.96905) (width 0.2) (layer "F.Cu") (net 14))
 (segment (start 64.7225 252.2225) (end 115.2225 252.2225) (width 0.2) (layer "F.Cu") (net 14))
 (segment (start 115.2225 252.2225) (end 119.9725 256.9725) (width 0.2) (layer "F.Cu") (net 14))
 (segment (start 119.9725 256.9725) (end 122.2695 256.9725) (width 0.2) (layer "F.Cu") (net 14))
 (segment (start 59.46905 246.96905) (end 64.7225 252.2225) (width 0.2) (layer "F.Cu") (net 14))
 (segment (start 73.76905 206.73095) (end 73.76905 218.75) (width 0.2) (layer "F.Cu") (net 13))
 (segment (start 73.76905 218.75) (end 73.76905 244.75) (width 0.2) (layer "F.Cu") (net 13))
 (segment (start 120.030186 256.4645) (end 122.2695 256.4645) (width 0.2) (layer "F.Cu") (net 13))
 (segment (start 73.76905 244.75) (end 80.73355 251.7145) (width 0.2) (layer "F.Cu") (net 13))
 (segment (start 80.73355 251.7145) (end 115.280186 251.7145) (width 0.2) (layer "F.Cu") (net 13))
 (segment (start 115.280186 251.7145) (end 120.030186 256.4645) (width 0.2) (layer "F.Cu") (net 13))
 (segment (start 89.25 179.26905) (end 89.25 245.25) (width 0.2) (layer "F.Cu") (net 12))
 (segment (start 95.2065 251.2065) (end 115.4565 251.2065) (width 0.2) (layer "F.Cu") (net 12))
 (segment (start 89.25 245.25) (end 95.2065 251.2065) (width 0.2) (layer "F.Cu") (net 12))
 (segment (start 103.76905 164.75) (end 89.25 179.26905) (width 0.2) (layer "F.Cu") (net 12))
 (segment (start 120.2065 255.9565) (end 122.2695 255.9565) (width 0.2) (layer "F.Cu") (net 12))
 (segment (start 115.4565 251.2065) (end 120.2065 255.9565) (width 0.2) (layer "F.Cu") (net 12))
 (segment (start 109.71755 250.6985) (end 115.514186 250.6985) (width 0.2) (layer "F.Cu") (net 4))
 (segment (start 103.76905 206.76905) (end 103.76905 218.75) (width 0.2) (layer "F.Cu") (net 4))
 (segment (start 103.76905 244.75) (end 109.71755 250.6985) (width 0.2) (layer "F.Cu") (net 4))
 (segment (start 103.76905 218.75) (end 103.76905 244.75) (width 0.2) (layer "F.Cu") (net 4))
 (segment (start 120.264186 255.4485) (end 122.2695 255.4485) (width 0.2) (layer "F.Cu") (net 4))
 (segment (start 115.514186 250.6985) (end 120.264186 255.4485) (width 0.2) (layer "F.Cu") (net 4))
 (segment (start 133.76905 164.75) (end 119.25 179.26905) (width 0.2) (layer "F.Cu") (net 11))
 (segment (start 119.25 179.26905) (end 119.25 244.25) (width 0.2) (layer "F.Cu") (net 11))
 (segment (start 122.968 247.968) (end 122.968 254.75) (width 0.2) (layer "F.Cu") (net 11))
 (segment (start 119.25 244.25) (end 122.968 247.968) (width 0.2) (layer "F.Cu") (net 11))
 (segment (start 133.76905 237.48095) (end 123.476 247.774) (width 0.2) (layer "F.Cu") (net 10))
 (segment (start 123.476 247.774) (end 123.476 254.75) (width 0.2) (layer "F.Cu") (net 10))
 (segment (start 133.76905 218.75) (end 133.76905 237.48095) (width 0.2) (layer "F.Cu") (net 10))
 (segment (start 123.984 248.266) (end 123.984 254.75) (width 0.2) (layer "F.Cu") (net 9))
 (segment (start 149.25 243.5) (end 147.25 245.5) (width 0.2) (layer "F.Cu") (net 9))
 (segment (start 126.75 245.5) (end 123.984 248.266) (width 0.2) (layer "F.Cu") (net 9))
 (segment (start 149.25 179.26905) (end 149.25 243.5) (width 0.2) (layer "F.Cu") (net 9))
 (segment (start 163.76905 164.75) (end 149.25 179.26905) (width 0.2) (layer "F.Cu") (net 9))
 (segment (start 147.25 245.5) (end 126.75 245.5) (width 0.2) (layer "F.Cu") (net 9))
 (segment (start 163.76905 234.48095) (end 152.25 246) (width 0.2) (layer "F.Cu") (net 8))
 (segment (start 152.25 246) (end 126.9333 246) (width 0.2) (layer "F.Cu") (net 8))
 (segment (start 126.9333 246) (end 124.492 248.4413) (width 0.2) (layer "F.Cu") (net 8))
 (segment (start 163.76905 218.75) (end 163.76905 234.48095) (width 0.2) (layer "F.Cu") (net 8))
 (segment (start 124.492 248.4413) (end 124.492 254.75) (width 0.2) (layer "F.Cu") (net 8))
 (segment (start 123.476 260.274) (end 122.75 261) (width 0.2) (layer "F.Cu") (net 2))
 (segment (start 123.476 258.687) (end 123.476 260.274) (width 0.2) (layer "F.Cu") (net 2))
 (segment (start 125 254.75) (end 125 254.1246) (width 0.2) (layer "F.Cu") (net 3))
 (segment (start 125 254.1246) (end 126.1246 253) (width 0.2) (layer "F.Cu") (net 3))
 (segment (start 126.1246 253) (end 129.5 253) (width 0.2) (layer "F.Cu") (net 3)))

